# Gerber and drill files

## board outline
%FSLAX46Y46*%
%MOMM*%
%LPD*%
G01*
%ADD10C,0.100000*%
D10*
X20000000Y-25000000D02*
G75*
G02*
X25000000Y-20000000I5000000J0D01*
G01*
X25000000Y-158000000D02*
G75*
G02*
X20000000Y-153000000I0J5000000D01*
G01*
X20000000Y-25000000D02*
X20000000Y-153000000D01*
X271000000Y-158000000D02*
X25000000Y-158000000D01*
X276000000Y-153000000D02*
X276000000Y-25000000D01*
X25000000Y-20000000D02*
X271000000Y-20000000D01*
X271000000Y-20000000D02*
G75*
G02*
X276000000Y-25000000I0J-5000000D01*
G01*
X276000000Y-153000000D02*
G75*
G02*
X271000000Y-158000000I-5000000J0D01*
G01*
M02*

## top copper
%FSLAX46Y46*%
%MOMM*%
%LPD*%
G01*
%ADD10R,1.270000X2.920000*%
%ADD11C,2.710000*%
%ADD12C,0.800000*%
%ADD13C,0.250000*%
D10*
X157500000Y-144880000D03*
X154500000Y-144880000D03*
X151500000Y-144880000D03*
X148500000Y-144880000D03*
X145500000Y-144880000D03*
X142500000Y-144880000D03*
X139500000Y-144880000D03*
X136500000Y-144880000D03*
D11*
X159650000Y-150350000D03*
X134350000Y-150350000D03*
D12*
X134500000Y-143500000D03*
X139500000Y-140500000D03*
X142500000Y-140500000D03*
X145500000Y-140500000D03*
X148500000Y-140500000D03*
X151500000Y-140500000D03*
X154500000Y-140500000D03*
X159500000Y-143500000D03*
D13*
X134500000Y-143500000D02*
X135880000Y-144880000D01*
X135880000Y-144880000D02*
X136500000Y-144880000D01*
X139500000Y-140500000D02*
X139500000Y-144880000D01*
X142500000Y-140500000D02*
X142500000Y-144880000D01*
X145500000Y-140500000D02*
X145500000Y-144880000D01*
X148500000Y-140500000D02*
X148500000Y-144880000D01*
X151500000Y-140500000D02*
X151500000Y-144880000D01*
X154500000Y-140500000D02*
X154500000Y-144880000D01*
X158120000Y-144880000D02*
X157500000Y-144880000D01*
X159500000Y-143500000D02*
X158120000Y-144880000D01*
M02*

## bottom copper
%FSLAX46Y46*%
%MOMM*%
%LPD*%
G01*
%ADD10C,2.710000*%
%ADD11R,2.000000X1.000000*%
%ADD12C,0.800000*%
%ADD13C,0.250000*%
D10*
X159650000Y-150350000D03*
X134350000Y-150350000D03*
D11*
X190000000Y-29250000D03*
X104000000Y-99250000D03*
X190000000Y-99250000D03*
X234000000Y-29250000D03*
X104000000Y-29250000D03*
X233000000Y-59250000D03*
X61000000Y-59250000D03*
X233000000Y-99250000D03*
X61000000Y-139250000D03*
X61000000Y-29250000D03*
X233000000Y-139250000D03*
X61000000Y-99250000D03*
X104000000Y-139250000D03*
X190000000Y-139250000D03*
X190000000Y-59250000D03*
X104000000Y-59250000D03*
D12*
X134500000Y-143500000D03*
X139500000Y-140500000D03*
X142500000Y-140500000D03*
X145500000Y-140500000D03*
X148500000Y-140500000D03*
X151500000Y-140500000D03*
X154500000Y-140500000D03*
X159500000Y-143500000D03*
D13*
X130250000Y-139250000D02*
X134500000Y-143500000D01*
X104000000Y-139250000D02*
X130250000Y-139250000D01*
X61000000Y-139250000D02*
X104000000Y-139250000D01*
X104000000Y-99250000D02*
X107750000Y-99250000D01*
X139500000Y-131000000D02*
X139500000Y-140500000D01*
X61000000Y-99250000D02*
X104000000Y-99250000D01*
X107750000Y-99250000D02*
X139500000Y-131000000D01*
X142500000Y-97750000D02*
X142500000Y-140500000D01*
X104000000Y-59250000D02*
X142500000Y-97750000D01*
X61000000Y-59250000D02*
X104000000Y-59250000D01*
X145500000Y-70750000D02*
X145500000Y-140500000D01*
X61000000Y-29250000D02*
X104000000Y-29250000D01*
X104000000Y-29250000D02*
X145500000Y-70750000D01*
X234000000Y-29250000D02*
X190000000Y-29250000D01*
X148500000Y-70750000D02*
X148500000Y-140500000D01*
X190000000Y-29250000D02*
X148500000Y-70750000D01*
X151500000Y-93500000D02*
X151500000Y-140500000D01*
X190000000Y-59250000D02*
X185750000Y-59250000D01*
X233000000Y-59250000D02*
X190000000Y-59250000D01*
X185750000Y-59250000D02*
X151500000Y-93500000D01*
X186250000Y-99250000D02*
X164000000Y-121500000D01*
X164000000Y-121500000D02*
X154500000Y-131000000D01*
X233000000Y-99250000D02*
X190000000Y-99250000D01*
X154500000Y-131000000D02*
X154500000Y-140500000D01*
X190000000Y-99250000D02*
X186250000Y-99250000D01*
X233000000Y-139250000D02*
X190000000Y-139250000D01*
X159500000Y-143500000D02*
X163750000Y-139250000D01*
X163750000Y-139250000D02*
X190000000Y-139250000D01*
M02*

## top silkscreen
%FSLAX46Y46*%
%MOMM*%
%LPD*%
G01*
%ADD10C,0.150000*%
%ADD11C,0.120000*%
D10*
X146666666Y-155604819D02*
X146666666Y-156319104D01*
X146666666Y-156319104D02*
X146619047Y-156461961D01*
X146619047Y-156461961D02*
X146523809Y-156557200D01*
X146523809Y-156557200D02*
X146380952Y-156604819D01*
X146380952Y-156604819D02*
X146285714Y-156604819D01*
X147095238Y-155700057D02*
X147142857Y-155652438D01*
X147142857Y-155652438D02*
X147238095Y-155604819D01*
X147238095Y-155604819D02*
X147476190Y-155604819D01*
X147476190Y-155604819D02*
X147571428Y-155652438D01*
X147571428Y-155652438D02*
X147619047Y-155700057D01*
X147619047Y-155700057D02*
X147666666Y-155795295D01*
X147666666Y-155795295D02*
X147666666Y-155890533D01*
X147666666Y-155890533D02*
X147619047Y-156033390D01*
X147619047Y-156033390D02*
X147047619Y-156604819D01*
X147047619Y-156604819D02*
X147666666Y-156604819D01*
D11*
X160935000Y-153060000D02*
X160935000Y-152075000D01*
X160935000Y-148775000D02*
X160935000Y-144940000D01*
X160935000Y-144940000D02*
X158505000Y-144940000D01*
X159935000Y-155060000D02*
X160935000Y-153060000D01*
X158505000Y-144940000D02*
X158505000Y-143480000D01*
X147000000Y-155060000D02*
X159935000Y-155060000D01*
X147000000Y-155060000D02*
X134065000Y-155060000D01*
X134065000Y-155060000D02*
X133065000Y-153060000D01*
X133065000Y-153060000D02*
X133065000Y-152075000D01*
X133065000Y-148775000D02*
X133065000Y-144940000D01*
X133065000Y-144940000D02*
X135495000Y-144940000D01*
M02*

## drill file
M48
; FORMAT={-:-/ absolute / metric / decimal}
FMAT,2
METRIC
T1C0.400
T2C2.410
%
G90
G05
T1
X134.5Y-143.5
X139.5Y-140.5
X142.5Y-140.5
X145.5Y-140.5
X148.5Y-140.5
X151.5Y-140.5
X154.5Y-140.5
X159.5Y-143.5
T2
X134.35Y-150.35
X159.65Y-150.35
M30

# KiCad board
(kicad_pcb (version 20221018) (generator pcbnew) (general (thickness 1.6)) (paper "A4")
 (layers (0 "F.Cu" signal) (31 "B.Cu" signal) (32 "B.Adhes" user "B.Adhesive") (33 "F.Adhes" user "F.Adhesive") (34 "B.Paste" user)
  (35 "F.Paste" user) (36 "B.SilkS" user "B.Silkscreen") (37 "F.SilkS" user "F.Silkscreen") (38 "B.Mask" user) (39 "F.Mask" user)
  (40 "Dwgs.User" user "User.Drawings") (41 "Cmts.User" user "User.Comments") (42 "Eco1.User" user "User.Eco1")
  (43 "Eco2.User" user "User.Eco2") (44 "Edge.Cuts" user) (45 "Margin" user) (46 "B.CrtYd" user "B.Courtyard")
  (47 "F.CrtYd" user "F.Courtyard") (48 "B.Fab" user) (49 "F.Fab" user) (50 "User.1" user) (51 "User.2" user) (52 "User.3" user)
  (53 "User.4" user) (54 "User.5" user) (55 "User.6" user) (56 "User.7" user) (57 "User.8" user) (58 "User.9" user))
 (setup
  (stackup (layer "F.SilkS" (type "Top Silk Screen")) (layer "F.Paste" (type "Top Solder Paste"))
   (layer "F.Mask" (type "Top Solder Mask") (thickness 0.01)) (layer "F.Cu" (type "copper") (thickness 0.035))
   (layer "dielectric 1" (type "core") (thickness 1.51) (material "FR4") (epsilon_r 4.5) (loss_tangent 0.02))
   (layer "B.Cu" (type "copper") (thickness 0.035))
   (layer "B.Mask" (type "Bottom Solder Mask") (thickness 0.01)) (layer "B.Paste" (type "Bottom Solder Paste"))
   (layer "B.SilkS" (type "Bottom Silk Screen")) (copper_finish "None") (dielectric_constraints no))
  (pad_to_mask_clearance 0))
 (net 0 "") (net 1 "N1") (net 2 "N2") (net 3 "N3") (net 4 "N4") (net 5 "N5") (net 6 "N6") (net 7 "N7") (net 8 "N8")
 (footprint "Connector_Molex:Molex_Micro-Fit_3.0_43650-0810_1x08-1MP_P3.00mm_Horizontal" (layer "F.Cu") (at 147 150 180)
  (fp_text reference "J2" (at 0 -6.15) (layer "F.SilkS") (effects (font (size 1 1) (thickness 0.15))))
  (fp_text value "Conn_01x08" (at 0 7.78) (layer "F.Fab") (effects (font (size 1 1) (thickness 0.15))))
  (fp_line (start -13.935 -3.06) (end -13.935 -2.075) (stroke (width 0.12) (type solid)) (layer "F.SilkS"))
  (fp_line (start -13.935 1.225) (end -13.935 5.06) (stroke (width 0.12) (type solid)) (layer "F.SilkS"))
  (fp_line (start -13.935 5.06) (end -11.505 5.06) (stroke (width 0.12) (type solid)) (layer "F.SilkS"))
  (fp_line (start -12.935 -5.06) (end -13.935 -3.06) (stroke (width 0.12) (type solid)) (layer "F.SilkS"))
  (fp_line (start -11.505 5.06) (end -11.505 6.52) (stroke (width 0.12) (type solid)) (layer "F.SilkS"))
  (fp_line (start 0 -5.06) (end -12.935 -5.06) (stroke (width 0.12) (type solid)) (layer "F.SilkS"))
  (fp_line (start 0 -5.06) (end 12.935 -5.06) (stroke (width 0.12) (type solid)) (layer "F.SilkS"))
  (fp_line (start 12.935 -5.06) (end 13.935 -3.06) (stroke (width 0.12) (type solid)) (layer "F.SilkS"))
  (fp_line (start 13.935 -3.06) (end 13.935 -2.075) (stroke (width 0.12) (type solid)) (layer "F.SilkS"))
  (fp_line (start 13.935 1.225) (end 13.935 5.06) (stroke (width 0.12) (type solid)) (layer "F.SilkS"))
  (fp_line (start 13.935 5.06) (end 11.505 5.06) (stroke (width 0.12) (type solid)) (layer "F.SilkS"))
  (pad "1" smd rect (at -10.5 5.12 180) (size 1.27 2.92) (layers "F.Cu" "F.Paste" "F.Mask") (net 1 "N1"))
  (pad "2" smd rect (at -7.5 5.12 180) (size 1.27 2.92) (layers "F.Cu" "F.Paste" "F.Mask") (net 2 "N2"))
  (pad "3" smd rect (at -4.5 5.12 180) (size 1.27 2.92) (layers "F.Cu" "F.Paste" "F.Mask") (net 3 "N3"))
  (pad "4" smd rect (at -1.5 5.12 180) (size 1.27 2.92) (layers "F.Cu" "F.Paste" "F.Mask") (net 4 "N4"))
  (pad "5" smd rect (at 1.5 5.12 180) (size 1.27 2.92) (layers "F.Cu" "F.Paste" "F.Mask") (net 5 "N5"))
  (pad "6" smd rect (at 4.5 5.12 180) (size 1.27 2.92) (layers "F.Cu" "F.Paste" "F.Mask") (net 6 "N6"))
  (pad "7" smd rect (at 7.5 5.12 180) (size 1.27 2.92) (layers "F.Cu" "F.Paste" "F.Mask") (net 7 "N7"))
  (pad "8" smd rect (at 10.5 5.12 180) (size 1.27 2.92) (layers "F.Cu" "F.Paste" "F.Mask") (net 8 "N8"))
  (pad "MP" thru_hole circle (at -12.65 -0.35 180) (size 2.71 2.71) (drill 2.41) (layers "*.Cu" "*.Mask"))
  (pad "MP" thru_hole circle (at 12.65 -0.35 180) (size 2.71 2.71) (drill 2.41) (layers "*.Cu" "*.Mask")))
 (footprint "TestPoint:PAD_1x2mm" (layer "B.Cu") (at 190 29.25 180)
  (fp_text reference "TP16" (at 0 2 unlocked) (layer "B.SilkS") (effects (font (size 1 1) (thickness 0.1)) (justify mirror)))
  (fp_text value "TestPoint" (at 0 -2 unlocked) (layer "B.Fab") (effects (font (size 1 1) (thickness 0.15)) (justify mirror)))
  (pad "1" smd rect (at 0 0 90) (size 1 2) (layers "B.Cu" "B.Paste" "B.Mask") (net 4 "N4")))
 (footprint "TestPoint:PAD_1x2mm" (layer "B.Cu") (at 104 99.25 180)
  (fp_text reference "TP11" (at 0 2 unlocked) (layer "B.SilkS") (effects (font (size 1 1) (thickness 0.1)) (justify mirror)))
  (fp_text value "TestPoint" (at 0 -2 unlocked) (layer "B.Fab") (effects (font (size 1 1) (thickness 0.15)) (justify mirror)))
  (pad "1" smd rect (at 0 0 90) (size 1 2) (layers "B.Cu" "B.Paste" "B.Mask") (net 7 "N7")))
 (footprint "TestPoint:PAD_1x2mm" (layer "B.Cu") (at 190 99.25 180)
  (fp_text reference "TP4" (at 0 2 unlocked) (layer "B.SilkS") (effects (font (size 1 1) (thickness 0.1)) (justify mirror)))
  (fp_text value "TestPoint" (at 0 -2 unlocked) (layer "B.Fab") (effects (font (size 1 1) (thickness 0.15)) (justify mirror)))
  (pad "1" smd rect (at 0 0 90) (size 1 2) (layers "B.Cu" "B.Paste" "B.Mask") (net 2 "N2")))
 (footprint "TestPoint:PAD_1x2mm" (layer "B.Cu") (at 234 29.25 180)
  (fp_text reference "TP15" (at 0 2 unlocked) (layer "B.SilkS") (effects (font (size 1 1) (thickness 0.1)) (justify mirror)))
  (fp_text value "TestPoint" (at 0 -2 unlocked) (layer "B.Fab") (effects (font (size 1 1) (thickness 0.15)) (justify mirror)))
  (pad "1" smd rect (at 0 0 90) (size 1 2) (layers "B.Cu" "B.Paste" "B.Mask") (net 4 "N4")))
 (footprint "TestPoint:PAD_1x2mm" (layer "B.Cu") (at 104 29.25 180)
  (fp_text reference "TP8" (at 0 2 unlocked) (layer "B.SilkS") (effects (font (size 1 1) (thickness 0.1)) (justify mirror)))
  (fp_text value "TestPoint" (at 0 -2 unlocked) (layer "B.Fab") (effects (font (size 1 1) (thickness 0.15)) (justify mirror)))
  (pad "1" smd rect (at 0 0 90) (size 1 2) (layers "B.Cu" "B.Paste" "B.Mask") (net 5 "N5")))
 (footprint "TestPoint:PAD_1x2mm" (layer "B.Cu") (at 233 59.25 180)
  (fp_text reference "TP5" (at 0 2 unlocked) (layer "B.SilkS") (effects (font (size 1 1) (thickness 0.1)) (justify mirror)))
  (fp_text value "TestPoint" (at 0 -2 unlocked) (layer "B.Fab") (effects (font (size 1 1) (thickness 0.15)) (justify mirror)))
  (pad "1" smd rect (at 0 0 90) (size 1 2) (layers "B.Cu" "B.Paste" "B.Mask") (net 3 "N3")))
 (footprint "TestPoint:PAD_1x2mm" (layer "B.Cu") (at 61 59.25 180)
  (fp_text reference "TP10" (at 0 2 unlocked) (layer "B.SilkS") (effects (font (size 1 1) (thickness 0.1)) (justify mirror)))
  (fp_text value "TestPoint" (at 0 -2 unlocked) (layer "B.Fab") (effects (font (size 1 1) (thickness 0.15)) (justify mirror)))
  (pad "1" smd rect (at 0 0 90) (size 1 2) (layers "B.Cu" "B.Paste" "B.Mask") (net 6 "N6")))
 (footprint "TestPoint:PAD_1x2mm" (layer "B.Cu") (at 233 99.25 180)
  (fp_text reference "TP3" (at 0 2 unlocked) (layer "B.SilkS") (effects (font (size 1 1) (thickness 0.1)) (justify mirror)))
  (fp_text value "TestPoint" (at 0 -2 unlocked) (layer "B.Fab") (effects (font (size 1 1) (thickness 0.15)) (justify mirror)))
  (pad "1" smd rect (at 0 0 90) (size 1 2) (layers "B.Cu" "B.Paste" "B.Mask") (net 2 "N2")))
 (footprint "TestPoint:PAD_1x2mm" (layer "B.Cu") (at 61 139.25 180)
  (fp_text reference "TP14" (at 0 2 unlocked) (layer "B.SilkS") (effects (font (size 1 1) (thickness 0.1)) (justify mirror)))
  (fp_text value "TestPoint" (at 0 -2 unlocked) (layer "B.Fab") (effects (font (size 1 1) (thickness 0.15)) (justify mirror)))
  (pad "1" smd rect (at 0 0 90) (size 1 2) (layers "B.Cu" "B.Paste" "B.Mask") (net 8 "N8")))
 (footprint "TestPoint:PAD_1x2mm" (layer "B.Cu") (at 61 29.25 180)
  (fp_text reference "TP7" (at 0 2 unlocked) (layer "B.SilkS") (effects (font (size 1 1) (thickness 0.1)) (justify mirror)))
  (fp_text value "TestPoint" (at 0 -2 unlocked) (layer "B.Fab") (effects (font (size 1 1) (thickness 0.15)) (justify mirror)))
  (pad "1" smd rect (at 0 0 90) (size 1 2) (layers "B.Cu" "B.Paste" "B.Mask") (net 5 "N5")))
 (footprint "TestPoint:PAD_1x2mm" (layer "B.Cu") (at 233 139.25 180)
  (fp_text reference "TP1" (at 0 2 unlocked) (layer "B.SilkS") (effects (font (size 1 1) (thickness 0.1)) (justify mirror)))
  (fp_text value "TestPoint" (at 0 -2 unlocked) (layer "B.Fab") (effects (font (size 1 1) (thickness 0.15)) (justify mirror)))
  (pad "1" smd rect (at 0 0 90) (size 1 2) (layers "B.Cu" "B.Paste" "B.Mask") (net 1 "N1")))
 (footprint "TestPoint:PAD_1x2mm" (layer "B.Cu") (at 61 99.25 180)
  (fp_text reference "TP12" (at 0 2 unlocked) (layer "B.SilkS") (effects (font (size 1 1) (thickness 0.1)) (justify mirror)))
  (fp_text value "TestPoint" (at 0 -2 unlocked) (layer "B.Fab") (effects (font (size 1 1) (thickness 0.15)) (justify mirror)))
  (pad "1" smd rect (at 0 0 90) (size 1 2) (layers "B.Cu" "B.Paste" "B.Mask") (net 7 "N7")))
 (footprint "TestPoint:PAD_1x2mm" (layer "B.Cu") (at 104 139.25 180)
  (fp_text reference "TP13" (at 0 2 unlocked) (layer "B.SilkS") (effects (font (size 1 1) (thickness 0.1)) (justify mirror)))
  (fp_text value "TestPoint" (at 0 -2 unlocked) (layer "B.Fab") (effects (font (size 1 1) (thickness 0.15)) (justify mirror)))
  (pad "1" smd rect (at 0 0 90) (size 1 2) (layers "B.Cu" "B.Paste" "B.Mask") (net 8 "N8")))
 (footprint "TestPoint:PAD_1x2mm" (layer "B.Cu") (at 190 139.25 180)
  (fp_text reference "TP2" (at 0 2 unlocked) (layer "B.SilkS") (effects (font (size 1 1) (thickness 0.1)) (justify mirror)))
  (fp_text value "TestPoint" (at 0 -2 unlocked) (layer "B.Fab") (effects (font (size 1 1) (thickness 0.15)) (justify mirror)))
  (pad "1" smd rect (at 0 0 90) (size 1 2) (layers "B.Cu" "B.Paste" "B.Mask") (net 1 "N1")))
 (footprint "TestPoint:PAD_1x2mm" (layer "B.Cu") (at 190 59.25 180)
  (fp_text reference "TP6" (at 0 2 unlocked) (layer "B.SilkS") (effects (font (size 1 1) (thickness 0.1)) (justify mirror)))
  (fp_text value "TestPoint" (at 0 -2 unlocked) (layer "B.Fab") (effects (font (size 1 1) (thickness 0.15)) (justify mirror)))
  (pad "1" smd rect (at 0 0 90) (size 1 2) (layers "B.Cu" "B.Paste" "B.Mask") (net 3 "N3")))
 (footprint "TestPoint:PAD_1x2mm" (layer "B.Cu") (at 104 59.25 180)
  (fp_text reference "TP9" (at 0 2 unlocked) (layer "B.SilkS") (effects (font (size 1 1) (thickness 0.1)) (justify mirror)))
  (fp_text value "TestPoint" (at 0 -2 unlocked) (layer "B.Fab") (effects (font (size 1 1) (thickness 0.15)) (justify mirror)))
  (pad "1" smd rect (at 0 0 90) (size 1 2) (layers "B.Cu" "B.Paste" "B.Mask") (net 6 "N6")))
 (gr_arc (start 20 25) (mid 21.464466 21.464466) (end 25 20) (stroke (width 0.1) (type default)) (layer "Edge.Cuts"))
 (gr_arc (start 25 158) (mid 21.464466 156.535534) (end 20 153) (stroke (width 0.1) (type default)) (layer "Edge.Cuts"))
 (gr_line (start 20 25) (end 20 153) (stroke (width 0.1) (type default)) (layer "Edge.Cuts"))
 (gr_line (start 271 158) (end 25 158) (stroke (width 0.1) (type default)) (layer "Edge.Cuts"))
 (gr_line (start 276 153) (end 276 25) (stroke (width 0.1) (type default)) (layer "Edge.Cuts"))
 (gr_line (start 25 20) (end 271 20) (stroke (width 0.1) (type default)) (layer "Edge.Cuts"))
 (gr_arc (start 271 20) (mid 274.535534 21.464466) (end 276 25) (stroke (width 0.1) (type default)) (layer "Edge.Cuts"))
 (gr_arc (start 276 153) (mid 274.535534 156.535534) (end 271 158) (stroke (width 0.1) (type default)) (layer "Edge.Cuts"))
 (segment (start 134.5 143.5) (end 135.88 144.88) (width 0.25) (layer "F.Cu") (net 8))
 (segment (start 135.88 144.88) (end 136.5 144.88) (width 0.25) (layer "F.Cu") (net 8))
 (via (at 134.5 143.5) (size 0.8) (drill 0.4) (layers "F.Cu" "B.Cu") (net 8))
 (segment (start 130.25 139.25) (end 134.5 143.5) (width 0.25) (layer "B.Cu") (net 8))
 (segment (start 104 139.25) (end 130.25 139.25) (width 0.25) (layer "B.Cu") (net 8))
 (segment (start 61 139.25) (end 104 139.25) (width 0.25) (layer "B.Cu") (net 8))
 (segment (start 139.5 140.5) (end 139.5 144.88) (width 0.25) (layer "F.Cu") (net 7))
 (via (at 139.5 140.5) (size 0.8) (drill 0.4) (layers "F.Cu" "B.Cu") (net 7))
 (segment (start 104 99.25) (end 107.75 99.25) (width 0.25) (layer "B.Cu") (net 7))
 (segment (start 139.5 131) (end 139.5 140.5) (width 0.25) (layer "B.Cu") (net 7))
 (segment (start 61 99.25) (end 104 99.25) (width 0.25) (layer "B.Cu") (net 7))
 (segment (start 107.75 99.25) (end 139.5 131) (width 0.25) (layer "B.Cu") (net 7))
 (segment (start 142.5 140.5) (end 142.5 144.88) (width 0.25) (layer "F.Cu") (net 6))
 (via (at 142.5 140.5) (size 0.8) (drill 0.4) (layers "F.Cu" "B.Cu") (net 6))
 (segment (start 142.5 97.75) (end 142.5 140.5) (width 0.25) (layer "B.Cu") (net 6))
 (segment (start 104 59.25) (end 142.5 97.75) (width 0.25) (layer "B.Cu") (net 6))
 (segment (start 61 59.25) (end 104 59.25) (width 0.25) (layer "B.Cu") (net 6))
 (segment (start 145.5 140.5) (end 145.5 144.88) (width 0.25) (layer "F.Cu") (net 5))
 (via (at 145.5 140.5) (size 0.8) (drill 0.4) (layers "F.Cu" "B.Cu") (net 5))
 (segment (start 145.5 70.75) (end 145.5 140.5) (width 0.25) (layer "B.Cu") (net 5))
 (segment (start 61 29.25) (end 104 29.25) (width 0.25) (layer "B.Cu") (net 5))
 (segment (start 104 29.25) (end 145.5 70.75) (width 0.25) (layer "B.Cu") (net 5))
 (segment (start 148.5 140.5) (end 148.5 144.88) (width 0.25) (layer "F.Cu") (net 4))
 (via (at 148.5 140.5) (size 0.8) (drill 0.4) (layers "F.Cu" "B.Cu") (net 4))
 (segment (start 234 29.25) (end 190 29.25) (width 0.25) (layer "B.Cu") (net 4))
 (segment (start 148.5 70.75) (end 148.5 140.5) (width 0.25) (layer "B.Cu") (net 4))
 (segment (start 190 29.25) (end 148.5 70.75) (width 0.25) (layer "B.Cu") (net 4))
 (segment (start 151.5 140.5) (end 151.5 144.88) (width 0.25) (layer "F.Cu") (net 3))
 (via (at 151.5 140.5) (size 0.8) (drill 0.4) (layers "F.Cu" "B.Cu") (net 3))
 (segment (start 151.5 93.5) (end 151.5 140.5) (width 0.25) (layer "B.Cu") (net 3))
 (segment (start 190 59.25) (end 185.75 59.25) (width 0.25) (layer "B.Cu") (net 3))
 (segment (start 233 59.25) (end 190 59.25) (width 0.25) (layer "B.Cu") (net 3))
 (segment (start 185.75 59.25) (end 151.5 93.5) (width 0.25) (layer "B.Cu") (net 3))
 (segment (start 154.5 140.5) (end 154.5 144.88) (width 0.25) (layer "F.Cu") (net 2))
 (via (at 154.5 140.5) (size 0.8) (drill 0.4) (layers "F.Cu" "B.Cu") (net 2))
 (segment (start 186.25 99.25) (end 164 121.5) (width 0.25) (layer "B.Cu") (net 2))
 (segment (start 164 121.5) (end 154.5 131) (width 0.25) (layer "B.Cu") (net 2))
 (segment (start 233 99.25) (end 190 99.25) (width 0.25) (layer "B.Cu") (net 2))
 (segment (start 154.5 131) (end 154.5 140.5) (width 0.25) (layer "B.Cu") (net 2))
 (segment (start 190 99.25) (end 186.25 99.25) (width 0.25) (layer "B.Cu") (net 2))
 (segment (start 158.12 144.88) (end 157.5 144.88) (width 0.25) (layer "F.Cu") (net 1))
 (segment (start 159.5 143.5) (end 158.12 144.88) (width 0.25) (layer "F.Cu") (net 1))
 (via (at 159.5 143.5) (size 0.8) (drill 0.4) (layers "F.Cu" "B.Cu") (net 1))
 (segment (start 233 139.25) (end 190 139.25) (width 0.25) (layer "B.Cu") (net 1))
 (segment (start 159.5 143.5) (end 163.75 139.25) (width 0.25) (layer "B.Cu") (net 1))
 (segment (start 163.75 139.25) (end 190 139.25) (width 0.25) (layer "B.Cu") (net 1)))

